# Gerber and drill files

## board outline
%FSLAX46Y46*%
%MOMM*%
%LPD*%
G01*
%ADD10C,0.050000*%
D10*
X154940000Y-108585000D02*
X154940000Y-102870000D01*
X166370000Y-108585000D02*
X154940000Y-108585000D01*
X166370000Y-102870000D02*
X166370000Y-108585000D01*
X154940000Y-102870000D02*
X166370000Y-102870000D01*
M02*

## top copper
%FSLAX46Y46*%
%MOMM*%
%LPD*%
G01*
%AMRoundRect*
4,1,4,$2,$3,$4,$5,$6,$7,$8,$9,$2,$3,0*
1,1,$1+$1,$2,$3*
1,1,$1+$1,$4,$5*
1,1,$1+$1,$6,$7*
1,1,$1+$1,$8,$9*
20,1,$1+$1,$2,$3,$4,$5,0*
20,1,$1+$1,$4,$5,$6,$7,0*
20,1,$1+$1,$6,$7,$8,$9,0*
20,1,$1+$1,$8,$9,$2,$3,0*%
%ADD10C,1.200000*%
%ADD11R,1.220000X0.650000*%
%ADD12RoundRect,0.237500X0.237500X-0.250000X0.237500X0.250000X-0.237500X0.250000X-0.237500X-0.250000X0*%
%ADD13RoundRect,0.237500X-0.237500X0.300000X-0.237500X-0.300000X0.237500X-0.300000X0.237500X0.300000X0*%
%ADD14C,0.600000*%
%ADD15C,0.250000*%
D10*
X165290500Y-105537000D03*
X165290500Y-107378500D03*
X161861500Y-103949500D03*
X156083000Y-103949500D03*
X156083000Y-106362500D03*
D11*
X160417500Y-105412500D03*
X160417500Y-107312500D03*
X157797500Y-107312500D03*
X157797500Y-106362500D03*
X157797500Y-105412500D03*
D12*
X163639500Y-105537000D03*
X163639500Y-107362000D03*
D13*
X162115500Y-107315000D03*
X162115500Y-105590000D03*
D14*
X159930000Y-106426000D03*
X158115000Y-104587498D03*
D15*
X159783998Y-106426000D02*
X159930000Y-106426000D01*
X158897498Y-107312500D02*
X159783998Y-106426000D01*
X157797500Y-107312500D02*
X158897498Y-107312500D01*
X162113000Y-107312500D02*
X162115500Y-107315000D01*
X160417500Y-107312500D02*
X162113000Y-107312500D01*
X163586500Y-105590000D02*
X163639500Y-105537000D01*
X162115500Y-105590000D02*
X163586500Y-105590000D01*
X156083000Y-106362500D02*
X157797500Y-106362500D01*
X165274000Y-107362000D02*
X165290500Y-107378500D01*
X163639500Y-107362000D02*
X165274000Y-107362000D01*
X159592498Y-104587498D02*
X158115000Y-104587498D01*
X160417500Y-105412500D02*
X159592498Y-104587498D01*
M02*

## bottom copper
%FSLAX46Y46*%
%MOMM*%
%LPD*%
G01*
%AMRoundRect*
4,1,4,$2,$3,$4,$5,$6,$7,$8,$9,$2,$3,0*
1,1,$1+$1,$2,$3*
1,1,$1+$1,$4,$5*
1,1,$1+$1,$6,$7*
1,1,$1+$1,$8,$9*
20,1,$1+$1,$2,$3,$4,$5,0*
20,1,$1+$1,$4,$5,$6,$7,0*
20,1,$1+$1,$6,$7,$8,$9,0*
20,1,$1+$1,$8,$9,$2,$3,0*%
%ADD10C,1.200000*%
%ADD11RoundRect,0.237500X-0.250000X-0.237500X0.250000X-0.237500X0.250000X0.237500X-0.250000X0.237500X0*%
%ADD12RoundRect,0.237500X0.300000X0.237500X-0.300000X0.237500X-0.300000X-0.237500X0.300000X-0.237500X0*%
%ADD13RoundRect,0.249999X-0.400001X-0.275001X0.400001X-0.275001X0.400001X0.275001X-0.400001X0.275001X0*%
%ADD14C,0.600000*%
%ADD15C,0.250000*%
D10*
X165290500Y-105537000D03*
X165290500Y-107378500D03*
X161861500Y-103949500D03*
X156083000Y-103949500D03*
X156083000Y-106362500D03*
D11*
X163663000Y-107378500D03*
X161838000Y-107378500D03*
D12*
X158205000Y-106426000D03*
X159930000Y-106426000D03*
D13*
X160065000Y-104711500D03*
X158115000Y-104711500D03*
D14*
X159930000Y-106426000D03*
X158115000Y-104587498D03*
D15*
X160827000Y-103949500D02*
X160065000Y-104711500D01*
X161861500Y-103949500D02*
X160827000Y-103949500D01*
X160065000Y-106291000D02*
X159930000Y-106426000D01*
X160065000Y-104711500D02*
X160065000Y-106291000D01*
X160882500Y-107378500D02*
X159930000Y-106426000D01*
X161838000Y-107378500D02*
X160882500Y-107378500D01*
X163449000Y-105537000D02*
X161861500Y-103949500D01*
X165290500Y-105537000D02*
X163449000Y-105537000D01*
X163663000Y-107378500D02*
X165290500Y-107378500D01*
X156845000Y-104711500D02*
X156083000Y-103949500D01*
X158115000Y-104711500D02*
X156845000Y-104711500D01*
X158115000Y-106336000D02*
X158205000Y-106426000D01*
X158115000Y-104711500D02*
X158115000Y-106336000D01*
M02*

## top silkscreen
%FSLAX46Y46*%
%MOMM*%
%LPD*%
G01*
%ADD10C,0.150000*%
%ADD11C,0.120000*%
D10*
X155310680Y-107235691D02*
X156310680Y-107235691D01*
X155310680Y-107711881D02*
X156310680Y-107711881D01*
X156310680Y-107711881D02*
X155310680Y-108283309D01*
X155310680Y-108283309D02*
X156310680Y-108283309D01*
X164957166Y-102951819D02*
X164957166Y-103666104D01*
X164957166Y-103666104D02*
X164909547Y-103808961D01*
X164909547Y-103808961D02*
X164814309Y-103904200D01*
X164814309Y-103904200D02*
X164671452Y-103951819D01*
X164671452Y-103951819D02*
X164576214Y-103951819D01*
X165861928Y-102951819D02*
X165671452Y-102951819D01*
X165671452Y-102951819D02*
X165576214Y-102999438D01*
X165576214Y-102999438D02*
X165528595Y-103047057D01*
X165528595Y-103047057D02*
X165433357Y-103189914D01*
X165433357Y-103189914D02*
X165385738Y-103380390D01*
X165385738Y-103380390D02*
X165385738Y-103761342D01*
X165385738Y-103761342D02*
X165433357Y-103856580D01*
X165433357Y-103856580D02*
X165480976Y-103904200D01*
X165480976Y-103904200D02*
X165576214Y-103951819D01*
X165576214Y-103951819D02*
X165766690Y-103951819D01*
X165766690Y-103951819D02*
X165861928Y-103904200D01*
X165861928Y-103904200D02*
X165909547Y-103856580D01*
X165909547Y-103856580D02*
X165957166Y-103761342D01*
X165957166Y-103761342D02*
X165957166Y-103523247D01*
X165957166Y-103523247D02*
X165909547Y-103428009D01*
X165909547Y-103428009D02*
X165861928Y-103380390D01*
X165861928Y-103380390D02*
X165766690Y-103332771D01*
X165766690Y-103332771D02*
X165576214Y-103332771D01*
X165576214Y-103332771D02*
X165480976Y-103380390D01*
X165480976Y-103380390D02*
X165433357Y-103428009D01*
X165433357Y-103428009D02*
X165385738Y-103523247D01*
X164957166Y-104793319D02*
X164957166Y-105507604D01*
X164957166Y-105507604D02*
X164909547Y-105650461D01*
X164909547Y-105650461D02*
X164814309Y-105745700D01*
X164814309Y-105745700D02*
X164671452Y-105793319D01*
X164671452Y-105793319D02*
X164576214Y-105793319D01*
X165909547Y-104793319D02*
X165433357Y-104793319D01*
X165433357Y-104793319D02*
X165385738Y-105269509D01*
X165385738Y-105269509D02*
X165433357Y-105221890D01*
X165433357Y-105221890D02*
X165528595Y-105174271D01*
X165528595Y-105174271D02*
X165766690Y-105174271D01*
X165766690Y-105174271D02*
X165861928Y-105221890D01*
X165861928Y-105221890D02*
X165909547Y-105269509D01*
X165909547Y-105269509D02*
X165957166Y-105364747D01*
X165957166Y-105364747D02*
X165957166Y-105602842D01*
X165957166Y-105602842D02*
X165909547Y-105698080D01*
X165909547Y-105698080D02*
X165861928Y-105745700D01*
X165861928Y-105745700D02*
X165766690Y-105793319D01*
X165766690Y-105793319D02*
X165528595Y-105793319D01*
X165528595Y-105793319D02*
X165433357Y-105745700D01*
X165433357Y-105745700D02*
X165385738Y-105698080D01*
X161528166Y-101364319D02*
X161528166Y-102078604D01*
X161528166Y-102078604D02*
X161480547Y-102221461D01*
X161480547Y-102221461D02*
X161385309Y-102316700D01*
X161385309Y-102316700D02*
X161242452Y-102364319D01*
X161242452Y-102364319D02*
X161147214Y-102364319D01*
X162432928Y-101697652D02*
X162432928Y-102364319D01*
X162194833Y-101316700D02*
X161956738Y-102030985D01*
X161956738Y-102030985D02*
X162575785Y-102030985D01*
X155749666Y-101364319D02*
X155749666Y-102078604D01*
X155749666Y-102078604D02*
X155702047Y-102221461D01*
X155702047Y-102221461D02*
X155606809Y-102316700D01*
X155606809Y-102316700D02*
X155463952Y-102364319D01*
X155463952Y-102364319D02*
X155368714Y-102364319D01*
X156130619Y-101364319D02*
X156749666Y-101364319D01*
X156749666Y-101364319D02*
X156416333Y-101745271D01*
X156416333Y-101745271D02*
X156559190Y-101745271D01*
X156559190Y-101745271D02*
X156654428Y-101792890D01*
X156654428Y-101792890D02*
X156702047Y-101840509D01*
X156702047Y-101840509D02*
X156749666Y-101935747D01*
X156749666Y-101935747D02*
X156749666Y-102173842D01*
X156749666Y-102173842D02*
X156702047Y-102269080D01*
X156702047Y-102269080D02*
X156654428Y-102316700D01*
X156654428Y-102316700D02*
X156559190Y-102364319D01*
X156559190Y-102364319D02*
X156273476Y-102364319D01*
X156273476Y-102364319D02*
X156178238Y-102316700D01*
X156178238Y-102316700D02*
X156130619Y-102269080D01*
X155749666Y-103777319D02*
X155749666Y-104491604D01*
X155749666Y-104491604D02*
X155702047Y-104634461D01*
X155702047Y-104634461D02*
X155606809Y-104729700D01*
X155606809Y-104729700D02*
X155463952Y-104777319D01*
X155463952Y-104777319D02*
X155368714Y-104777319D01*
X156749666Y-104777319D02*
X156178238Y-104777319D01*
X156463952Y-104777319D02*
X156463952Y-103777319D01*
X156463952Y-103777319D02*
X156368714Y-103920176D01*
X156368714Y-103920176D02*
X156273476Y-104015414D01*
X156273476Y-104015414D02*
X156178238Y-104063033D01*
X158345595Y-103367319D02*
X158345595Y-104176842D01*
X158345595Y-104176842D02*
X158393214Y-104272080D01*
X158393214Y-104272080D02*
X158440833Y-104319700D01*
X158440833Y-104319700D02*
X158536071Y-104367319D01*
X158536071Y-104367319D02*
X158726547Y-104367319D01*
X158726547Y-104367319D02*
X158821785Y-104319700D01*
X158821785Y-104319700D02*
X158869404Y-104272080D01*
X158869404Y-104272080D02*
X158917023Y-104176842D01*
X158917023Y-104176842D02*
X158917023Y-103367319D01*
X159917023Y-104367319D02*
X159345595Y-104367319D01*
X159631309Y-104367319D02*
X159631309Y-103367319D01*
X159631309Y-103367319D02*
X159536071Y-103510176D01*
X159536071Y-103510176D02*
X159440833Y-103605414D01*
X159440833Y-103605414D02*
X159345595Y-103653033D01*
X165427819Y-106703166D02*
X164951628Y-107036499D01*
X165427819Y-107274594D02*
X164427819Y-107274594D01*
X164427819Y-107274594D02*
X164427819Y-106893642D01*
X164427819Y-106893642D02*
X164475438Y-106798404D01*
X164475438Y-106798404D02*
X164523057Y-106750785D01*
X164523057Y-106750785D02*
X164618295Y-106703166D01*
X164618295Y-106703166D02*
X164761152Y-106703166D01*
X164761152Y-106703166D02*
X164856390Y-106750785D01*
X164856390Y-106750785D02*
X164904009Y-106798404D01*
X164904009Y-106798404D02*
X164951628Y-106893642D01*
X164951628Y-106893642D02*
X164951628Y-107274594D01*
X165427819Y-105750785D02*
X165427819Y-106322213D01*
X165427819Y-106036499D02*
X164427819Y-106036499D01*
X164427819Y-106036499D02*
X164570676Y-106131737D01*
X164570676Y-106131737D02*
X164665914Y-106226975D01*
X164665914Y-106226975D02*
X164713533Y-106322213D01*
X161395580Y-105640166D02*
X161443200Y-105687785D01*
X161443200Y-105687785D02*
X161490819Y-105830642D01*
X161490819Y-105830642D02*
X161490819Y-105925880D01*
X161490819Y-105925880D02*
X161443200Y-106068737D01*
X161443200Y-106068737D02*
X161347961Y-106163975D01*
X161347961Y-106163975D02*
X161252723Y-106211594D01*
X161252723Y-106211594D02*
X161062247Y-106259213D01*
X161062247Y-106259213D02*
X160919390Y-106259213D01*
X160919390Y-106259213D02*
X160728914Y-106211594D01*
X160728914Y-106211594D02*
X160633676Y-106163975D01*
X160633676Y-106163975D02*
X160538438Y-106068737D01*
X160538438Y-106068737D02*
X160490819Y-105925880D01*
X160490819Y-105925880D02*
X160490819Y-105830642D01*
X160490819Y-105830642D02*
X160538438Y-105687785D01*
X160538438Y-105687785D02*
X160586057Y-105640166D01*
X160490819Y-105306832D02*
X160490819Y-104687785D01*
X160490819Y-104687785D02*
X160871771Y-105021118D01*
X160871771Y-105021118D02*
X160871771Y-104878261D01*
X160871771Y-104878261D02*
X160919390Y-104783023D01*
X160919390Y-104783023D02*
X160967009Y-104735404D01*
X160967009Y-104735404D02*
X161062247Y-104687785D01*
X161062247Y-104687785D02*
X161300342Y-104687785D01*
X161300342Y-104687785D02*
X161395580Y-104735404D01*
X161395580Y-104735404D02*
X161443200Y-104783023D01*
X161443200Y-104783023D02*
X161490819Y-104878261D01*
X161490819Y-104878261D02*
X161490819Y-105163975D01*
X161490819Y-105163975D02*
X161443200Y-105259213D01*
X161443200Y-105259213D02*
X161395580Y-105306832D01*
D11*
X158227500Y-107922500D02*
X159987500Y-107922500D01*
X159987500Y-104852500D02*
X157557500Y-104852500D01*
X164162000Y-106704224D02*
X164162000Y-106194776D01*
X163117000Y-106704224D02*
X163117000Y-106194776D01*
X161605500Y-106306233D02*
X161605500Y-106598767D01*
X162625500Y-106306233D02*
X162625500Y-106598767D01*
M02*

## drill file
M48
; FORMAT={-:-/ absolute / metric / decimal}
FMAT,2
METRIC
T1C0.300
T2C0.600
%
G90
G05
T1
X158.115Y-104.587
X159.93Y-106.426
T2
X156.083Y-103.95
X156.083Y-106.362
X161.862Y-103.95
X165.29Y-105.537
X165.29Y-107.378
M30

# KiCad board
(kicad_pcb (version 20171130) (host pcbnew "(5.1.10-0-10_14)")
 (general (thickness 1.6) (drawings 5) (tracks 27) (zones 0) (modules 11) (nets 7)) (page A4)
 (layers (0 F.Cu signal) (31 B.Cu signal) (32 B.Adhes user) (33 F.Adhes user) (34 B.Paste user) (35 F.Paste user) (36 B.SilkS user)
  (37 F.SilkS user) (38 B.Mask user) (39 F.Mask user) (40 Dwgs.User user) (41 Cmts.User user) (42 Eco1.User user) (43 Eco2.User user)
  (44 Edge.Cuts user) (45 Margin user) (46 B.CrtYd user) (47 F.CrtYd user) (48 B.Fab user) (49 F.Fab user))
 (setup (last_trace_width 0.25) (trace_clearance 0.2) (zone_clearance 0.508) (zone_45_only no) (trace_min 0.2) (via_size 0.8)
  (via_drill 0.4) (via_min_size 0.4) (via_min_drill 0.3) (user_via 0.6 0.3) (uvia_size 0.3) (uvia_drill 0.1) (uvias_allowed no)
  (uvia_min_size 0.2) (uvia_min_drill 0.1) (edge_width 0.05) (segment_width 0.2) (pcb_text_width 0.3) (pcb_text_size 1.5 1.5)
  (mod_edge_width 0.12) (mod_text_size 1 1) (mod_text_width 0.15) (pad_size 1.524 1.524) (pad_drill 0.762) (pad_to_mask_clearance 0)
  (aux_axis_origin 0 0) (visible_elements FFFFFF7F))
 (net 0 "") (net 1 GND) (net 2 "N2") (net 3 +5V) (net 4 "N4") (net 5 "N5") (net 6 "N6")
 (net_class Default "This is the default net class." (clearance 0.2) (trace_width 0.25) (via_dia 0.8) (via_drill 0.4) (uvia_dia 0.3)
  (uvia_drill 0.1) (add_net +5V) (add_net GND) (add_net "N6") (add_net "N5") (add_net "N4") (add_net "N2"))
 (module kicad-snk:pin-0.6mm (layer F.Cu) (at 165.2905 102.997)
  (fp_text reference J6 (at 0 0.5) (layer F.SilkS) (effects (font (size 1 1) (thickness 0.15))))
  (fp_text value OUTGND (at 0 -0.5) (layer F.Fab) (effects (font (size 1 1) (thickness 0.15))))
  (pad 1 thru_hole circle (at 0 2.54) (size 1.2 1.2) (drill 0.6) (layers *.Cu *.Mask) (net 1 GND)))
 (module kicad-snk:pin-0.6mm (layer F.Cu) (at 165.2905 104.8385)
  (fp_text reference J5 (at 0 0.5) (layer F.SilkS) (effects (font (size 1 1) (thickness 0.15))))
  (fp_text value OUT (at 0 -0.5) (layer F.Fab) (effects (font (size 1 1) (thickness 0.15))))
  (pad 1 thru_hole circle (at 0 2.54) (size 1.2 1.2) (drill 0.6) (layers *.Cu *.Mask) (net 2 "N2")))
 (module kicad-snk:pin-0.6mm (layer F.Cu) (at 161.8615 101.4095)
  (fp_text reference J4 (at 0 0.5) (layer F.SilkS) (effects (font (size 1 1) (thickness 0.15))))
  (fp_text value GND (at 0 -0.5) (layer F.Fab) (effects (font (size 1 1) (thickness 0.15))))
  (pad 1 thru_hole circle (at 0 2.54) (size 1.2 1.2) (drill 0.6) (layers *.Cu *.Mask) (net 1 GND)))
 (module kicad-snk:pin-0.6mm (layer F.Cu) (at 156.083 101.4095)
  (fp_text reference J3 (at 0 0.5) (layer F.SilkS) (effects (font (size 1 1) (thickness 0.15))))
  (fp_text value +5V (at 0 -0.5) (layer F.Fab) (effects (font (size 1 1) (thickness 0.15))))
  (pad 1 thru_hole circle (at 0 2.54) (size 1.2 1.2) (drill 0.6) (layers *.Cu *.Mask) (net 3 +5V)))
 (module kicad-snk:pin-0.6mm (layer F.Cu) (at 156.083 103.8225)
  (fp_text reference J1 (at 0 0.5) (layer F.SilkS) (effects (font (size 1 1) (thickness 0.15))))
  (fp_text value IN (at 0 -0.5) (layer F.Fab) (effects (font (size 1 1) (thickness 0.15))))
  (pad 1 thru_hole circle (at 0 2.54) (size 1.2 1.2) (drill 0.6) (layers *.Cu *.Mask) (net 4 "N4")))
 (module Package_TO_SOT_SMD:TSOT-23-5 (layer F.Cu) (at 159.1075 106.3625)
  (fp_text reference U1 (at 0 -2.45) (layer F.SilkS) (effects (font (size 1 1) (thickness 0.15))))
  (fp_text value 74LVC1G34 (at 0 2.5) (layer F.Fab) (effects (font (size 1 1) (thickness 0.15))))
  (fp_line (start -0.88 1.56) (end 0.88 1.56) (layer F.SilkS) (width 0.12))
  (fp_line (start 0.88 -1.51) (end -1.55 -1.51) (layer F.SilkS) (width 0.12))
  (pad 5 smd rect (at 1.31 -0.95) (size 1.22 0.65) (layers F.Cu F.Paste F.Mask) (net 3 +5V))
  (pad 4 smd rect (at 1.31 0.95) (size 1.22 0.65) (layers F.Cu F.Paste F.Mask) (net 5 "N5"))
  (pad 3 smd rect (at -1.31 0.95) (size 1.22 0.65) (layers F.Cu F.Paste F.Mask) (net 1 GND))
  (pad 2 smd rect (at -1.31 0) (size 1.22 0.65) (layers F.Cu F.Paste F.Mask) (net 4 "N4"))
  (pad 1 smd rect (at -1.31 -0.95) (size 1.22 0.65) (layers F.Cu F.Paste F.Mask)))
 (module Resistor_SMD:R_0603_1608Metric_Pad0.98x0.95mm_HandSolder (layer B.Cu) (at 162.7505 107.3785)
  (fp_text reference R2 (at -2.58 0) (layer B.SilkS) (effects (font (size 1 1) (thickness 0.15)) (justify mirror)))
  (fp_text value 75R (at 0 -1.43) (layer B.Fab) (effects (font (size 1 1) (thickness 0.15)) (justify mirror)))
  (pad 2 smd roundrect (at 0.9125 0) (size 0.975 0.95) (layers B.Cu B.Paste B.Mask) (roundrect_rratio 0.25) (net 2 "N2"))
  (pad 1 smd roundrect (at -0.9125 0) (size 0.975 0.95) (layers B.Cu B.Paste B.Mask) (roundrect_rratio 0.25) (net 1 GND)))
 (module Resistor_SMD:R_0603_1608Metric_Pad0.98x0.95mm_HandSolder (layer F.Cu) (at 163.6395 106.4495 90)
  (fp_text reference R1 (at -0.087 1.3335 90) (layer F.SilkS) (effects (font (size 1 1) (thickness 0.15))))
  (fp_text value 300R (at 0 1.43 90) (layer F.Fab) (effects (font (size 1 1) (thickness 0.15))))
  (fp_line (start -0.254724 0.5225) (end 0.254724 0.5225) (layer F.SilkS) (width 0.12))
  (fp_line (start -0.254724 -0.5225) (end 0.254724 -0.5225) (layer F.SilkS) (width 0.12))
  (pad 2 smd roundrect (at 0.9125 0 90) (size 0.975 0.95) (layers F.Cu F.Paste F.Mask) (roundrect_rratio 0.25) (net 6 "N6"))
  (pad 1 smd roundrect (at -0.9125 0 90) (size 0.975 0.95) (layers F.Cu F.Paste F.Mask) (roundrect_rratio 0.25) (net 2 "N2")))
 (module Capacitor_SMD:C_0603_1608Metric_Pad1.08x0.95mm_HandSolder (layer F.Cu) (at 162.1155 106.4525 270)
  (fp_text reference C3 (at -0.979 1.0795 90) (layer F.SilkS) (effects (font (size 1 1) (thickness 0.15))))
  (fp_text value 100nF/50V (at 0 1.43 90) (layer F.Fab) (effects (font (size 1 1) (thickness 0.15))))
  (fp_line (start -0.146267 0.51) (end 0.146267 0.51) (layer F.SilkS) (width 0.12))
  (fp_line (start -0.146267 -0.51) (end 0.146267 -0.51) (layer F.SilkS) (width 0.12))
  (pad 2 smd roundrect (at 0.8625 0 270) (size 1.075 0.95) (layers F.Cu F.Paste F.Mask) (roundrect_rratio 0.25) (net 5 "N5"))
  (pad 1 smd roundrect (at -0.8625 0 270) (size 1.075 0.95) (layers F.Cu F.Paste F.Mask) (roundrect_rratio 0.25) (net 6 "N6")))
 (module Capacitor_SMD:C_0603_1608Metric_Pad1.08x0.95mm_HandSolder (layer B.Cu) (at 159.0675 106.426 180)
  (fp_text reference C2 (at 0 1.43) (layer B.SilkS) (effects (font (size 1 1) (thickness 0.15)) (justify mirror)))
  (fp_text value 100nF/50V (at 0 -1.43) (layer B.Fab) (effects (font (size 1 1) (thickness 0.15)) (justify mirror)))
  (pad 2 smd roundrect (at 0.8625 0 180) (size 1.075 0.95) (layers B.Cu B.Paste B.Mask) (roundrect_rratio 0.25) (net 3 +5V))
  (pad 1 smd roundrect (at -0.8625 0 180) (size 1.075 0.95) (layers B.Cu B.Paste B.Mask) (roundrect_rratio 0.25) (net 1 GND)))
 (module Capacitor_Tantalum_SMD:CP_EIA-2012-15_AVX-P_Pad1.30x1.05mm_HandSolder (layer B.Cu) (at 159.09 104.7115)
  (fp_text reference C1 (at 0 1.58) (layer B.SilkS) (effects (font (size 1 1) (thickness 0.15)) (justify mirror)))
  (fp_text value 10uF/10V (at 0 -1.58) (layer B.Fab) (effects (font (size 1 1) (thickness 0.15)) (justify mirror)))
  (pad 2 smd roundrect (at 0.975 0) (size 1.3 1.05) (layers B.Cu B.Paste B.Mask) (roundrect_rratio 0.2380942857142857) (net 1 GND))
  (pad 1 smd roundrect (at -0.975 0) (size 1.3 1.05) (layers B.Cu B.Paste B.Mask) (roundrect_rratio 0.2380942857142857) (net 3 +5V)))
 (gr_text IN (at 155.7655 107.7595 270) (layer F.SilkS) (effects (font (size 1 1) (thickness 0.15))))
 (gr_line (start 154.94 108.585) (end 154.94 102.87) (layer Edge.Cuts) (width 0.05))
 (gr_line (start 166.37 108.585) (end 154.94 108.585) (layer Edge.Cuts) (width 0.05))
 (gr_line (start 166.37 102.87) (end 166.37 108.585) (layer Edge.Cuts) (width 0.05))
 (gr_line (start 154.94 102.87) (end 166.37 102.87) (layer Edge.Cuts) (width 0.05))
 (segment (start 160.827 103.9495) (end 160.065 104.7115) (width 0.25) (layer B.Cu) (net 1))
 (segment (start 161.8615 103.9495) (end 160.827 103.9495) (width 0.25) (layer B.Cu) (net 1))
 (segment (start 160.065 106.291) (end 159.93 106.426) (width 0.25) (layer B.Cu) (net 1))
 (segment (start 160.065 104.7115) (end 160.065 106.291) (width 0.25) (layer B.Cu) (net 1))
 (segment (start 160.8825 107.3785) (end 159.93 106.426) (width 0.25) (layer B.Cu) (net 1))
 (segment (start 161.838 107.3785) (end 160.8825 107.3785) (width 0.25) (layer B.Cu) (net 1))
 (via (at 159.93 106.426) (size 0.6) (drill 0.3) (layers F.Cu B.Cu) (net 1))
 (segment (start 159.783998 106.426) (end 159.93 106.426) (width 0.25) (layer F.Cu) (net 1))
 (segment (start 158.897498 107.3125) (end 159.783998 106.426) (width 0.25) (layer F.Cu) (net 1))
 (segment (start 157.7975 107.3125) (end 158.897498 107.3125) (width 0.25) (layer F.Cu) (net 1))
 (segment (start 163.449 105.537) (end 161.8615 103.9495) (width 0.25) (layer B.Cu) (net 1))
 (segment (start 165.2905 105.537) (end 163.449 105.537) (width 0.25) (layer B.Cu) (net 1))
 (segment (start 162.113 107.3125) (end 162.1155 107.315) (width 0.25) (layer F.Cu) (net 5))
 (segment (start 160.4175 107.3125) (end 162.113 107.3125) (width 0.25) (layer F.Cu) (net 5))
 (segment (start 163.5865 105.59) (end 163.6395 105.537) (width 0.25) (layer F.Cu) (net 6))
 (segment (start 162.1155 105.59) (end 163.5865 105.59) (width 0.25) (layer F.Cu) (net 6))
 (segment (start 156.083 106.3625) (end 157.7975 106.3625) (width 0.25) (layer F.Cu) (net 4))
 (segment (start 165.274 107.362) (end 165.2905 107.3785) (width 0.25) (layer F.Cu) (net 2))
 (segment (start 163.6395 107.362) (end 165.274 107.362) (width 0.25) (layer F.Cu) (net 2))
 (segment (start 163.663 107.3785) (end 165.2905 107.3785) (width 0.25) (layer B.Cu) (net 2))
 (segment (start 156.845 104.7115) (end 156.083 103.9495) (width 0.25) (layer B.Cu) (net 3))
 (segment (start 158.115 104.7115) (end 156.845 104.7115) (width 0.25) (layer B.Cu) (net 3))
 (segment (start 158.115 106.336) (end 158.205 106.426) (width 0.25) (layer B.Cu) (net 3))
 (segment (start 158.115 104.7115) (end 158.115 106.336) (width 0.25) (layer B.Cu) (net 3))
 (via (at 158.115 104.587498) (size 0.6) (drill 0.3) (layers F.Cu B.Cu) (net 3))
 (segment (start 159.592498 104.587498) (end 158.115 104.587498) (width 0.25) (layer F.Cu) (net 3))
 (segment (start 160.4175 105.4125) (end 159.592498 104.587498) (width 0.25) (layer F.Cu) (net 3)))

